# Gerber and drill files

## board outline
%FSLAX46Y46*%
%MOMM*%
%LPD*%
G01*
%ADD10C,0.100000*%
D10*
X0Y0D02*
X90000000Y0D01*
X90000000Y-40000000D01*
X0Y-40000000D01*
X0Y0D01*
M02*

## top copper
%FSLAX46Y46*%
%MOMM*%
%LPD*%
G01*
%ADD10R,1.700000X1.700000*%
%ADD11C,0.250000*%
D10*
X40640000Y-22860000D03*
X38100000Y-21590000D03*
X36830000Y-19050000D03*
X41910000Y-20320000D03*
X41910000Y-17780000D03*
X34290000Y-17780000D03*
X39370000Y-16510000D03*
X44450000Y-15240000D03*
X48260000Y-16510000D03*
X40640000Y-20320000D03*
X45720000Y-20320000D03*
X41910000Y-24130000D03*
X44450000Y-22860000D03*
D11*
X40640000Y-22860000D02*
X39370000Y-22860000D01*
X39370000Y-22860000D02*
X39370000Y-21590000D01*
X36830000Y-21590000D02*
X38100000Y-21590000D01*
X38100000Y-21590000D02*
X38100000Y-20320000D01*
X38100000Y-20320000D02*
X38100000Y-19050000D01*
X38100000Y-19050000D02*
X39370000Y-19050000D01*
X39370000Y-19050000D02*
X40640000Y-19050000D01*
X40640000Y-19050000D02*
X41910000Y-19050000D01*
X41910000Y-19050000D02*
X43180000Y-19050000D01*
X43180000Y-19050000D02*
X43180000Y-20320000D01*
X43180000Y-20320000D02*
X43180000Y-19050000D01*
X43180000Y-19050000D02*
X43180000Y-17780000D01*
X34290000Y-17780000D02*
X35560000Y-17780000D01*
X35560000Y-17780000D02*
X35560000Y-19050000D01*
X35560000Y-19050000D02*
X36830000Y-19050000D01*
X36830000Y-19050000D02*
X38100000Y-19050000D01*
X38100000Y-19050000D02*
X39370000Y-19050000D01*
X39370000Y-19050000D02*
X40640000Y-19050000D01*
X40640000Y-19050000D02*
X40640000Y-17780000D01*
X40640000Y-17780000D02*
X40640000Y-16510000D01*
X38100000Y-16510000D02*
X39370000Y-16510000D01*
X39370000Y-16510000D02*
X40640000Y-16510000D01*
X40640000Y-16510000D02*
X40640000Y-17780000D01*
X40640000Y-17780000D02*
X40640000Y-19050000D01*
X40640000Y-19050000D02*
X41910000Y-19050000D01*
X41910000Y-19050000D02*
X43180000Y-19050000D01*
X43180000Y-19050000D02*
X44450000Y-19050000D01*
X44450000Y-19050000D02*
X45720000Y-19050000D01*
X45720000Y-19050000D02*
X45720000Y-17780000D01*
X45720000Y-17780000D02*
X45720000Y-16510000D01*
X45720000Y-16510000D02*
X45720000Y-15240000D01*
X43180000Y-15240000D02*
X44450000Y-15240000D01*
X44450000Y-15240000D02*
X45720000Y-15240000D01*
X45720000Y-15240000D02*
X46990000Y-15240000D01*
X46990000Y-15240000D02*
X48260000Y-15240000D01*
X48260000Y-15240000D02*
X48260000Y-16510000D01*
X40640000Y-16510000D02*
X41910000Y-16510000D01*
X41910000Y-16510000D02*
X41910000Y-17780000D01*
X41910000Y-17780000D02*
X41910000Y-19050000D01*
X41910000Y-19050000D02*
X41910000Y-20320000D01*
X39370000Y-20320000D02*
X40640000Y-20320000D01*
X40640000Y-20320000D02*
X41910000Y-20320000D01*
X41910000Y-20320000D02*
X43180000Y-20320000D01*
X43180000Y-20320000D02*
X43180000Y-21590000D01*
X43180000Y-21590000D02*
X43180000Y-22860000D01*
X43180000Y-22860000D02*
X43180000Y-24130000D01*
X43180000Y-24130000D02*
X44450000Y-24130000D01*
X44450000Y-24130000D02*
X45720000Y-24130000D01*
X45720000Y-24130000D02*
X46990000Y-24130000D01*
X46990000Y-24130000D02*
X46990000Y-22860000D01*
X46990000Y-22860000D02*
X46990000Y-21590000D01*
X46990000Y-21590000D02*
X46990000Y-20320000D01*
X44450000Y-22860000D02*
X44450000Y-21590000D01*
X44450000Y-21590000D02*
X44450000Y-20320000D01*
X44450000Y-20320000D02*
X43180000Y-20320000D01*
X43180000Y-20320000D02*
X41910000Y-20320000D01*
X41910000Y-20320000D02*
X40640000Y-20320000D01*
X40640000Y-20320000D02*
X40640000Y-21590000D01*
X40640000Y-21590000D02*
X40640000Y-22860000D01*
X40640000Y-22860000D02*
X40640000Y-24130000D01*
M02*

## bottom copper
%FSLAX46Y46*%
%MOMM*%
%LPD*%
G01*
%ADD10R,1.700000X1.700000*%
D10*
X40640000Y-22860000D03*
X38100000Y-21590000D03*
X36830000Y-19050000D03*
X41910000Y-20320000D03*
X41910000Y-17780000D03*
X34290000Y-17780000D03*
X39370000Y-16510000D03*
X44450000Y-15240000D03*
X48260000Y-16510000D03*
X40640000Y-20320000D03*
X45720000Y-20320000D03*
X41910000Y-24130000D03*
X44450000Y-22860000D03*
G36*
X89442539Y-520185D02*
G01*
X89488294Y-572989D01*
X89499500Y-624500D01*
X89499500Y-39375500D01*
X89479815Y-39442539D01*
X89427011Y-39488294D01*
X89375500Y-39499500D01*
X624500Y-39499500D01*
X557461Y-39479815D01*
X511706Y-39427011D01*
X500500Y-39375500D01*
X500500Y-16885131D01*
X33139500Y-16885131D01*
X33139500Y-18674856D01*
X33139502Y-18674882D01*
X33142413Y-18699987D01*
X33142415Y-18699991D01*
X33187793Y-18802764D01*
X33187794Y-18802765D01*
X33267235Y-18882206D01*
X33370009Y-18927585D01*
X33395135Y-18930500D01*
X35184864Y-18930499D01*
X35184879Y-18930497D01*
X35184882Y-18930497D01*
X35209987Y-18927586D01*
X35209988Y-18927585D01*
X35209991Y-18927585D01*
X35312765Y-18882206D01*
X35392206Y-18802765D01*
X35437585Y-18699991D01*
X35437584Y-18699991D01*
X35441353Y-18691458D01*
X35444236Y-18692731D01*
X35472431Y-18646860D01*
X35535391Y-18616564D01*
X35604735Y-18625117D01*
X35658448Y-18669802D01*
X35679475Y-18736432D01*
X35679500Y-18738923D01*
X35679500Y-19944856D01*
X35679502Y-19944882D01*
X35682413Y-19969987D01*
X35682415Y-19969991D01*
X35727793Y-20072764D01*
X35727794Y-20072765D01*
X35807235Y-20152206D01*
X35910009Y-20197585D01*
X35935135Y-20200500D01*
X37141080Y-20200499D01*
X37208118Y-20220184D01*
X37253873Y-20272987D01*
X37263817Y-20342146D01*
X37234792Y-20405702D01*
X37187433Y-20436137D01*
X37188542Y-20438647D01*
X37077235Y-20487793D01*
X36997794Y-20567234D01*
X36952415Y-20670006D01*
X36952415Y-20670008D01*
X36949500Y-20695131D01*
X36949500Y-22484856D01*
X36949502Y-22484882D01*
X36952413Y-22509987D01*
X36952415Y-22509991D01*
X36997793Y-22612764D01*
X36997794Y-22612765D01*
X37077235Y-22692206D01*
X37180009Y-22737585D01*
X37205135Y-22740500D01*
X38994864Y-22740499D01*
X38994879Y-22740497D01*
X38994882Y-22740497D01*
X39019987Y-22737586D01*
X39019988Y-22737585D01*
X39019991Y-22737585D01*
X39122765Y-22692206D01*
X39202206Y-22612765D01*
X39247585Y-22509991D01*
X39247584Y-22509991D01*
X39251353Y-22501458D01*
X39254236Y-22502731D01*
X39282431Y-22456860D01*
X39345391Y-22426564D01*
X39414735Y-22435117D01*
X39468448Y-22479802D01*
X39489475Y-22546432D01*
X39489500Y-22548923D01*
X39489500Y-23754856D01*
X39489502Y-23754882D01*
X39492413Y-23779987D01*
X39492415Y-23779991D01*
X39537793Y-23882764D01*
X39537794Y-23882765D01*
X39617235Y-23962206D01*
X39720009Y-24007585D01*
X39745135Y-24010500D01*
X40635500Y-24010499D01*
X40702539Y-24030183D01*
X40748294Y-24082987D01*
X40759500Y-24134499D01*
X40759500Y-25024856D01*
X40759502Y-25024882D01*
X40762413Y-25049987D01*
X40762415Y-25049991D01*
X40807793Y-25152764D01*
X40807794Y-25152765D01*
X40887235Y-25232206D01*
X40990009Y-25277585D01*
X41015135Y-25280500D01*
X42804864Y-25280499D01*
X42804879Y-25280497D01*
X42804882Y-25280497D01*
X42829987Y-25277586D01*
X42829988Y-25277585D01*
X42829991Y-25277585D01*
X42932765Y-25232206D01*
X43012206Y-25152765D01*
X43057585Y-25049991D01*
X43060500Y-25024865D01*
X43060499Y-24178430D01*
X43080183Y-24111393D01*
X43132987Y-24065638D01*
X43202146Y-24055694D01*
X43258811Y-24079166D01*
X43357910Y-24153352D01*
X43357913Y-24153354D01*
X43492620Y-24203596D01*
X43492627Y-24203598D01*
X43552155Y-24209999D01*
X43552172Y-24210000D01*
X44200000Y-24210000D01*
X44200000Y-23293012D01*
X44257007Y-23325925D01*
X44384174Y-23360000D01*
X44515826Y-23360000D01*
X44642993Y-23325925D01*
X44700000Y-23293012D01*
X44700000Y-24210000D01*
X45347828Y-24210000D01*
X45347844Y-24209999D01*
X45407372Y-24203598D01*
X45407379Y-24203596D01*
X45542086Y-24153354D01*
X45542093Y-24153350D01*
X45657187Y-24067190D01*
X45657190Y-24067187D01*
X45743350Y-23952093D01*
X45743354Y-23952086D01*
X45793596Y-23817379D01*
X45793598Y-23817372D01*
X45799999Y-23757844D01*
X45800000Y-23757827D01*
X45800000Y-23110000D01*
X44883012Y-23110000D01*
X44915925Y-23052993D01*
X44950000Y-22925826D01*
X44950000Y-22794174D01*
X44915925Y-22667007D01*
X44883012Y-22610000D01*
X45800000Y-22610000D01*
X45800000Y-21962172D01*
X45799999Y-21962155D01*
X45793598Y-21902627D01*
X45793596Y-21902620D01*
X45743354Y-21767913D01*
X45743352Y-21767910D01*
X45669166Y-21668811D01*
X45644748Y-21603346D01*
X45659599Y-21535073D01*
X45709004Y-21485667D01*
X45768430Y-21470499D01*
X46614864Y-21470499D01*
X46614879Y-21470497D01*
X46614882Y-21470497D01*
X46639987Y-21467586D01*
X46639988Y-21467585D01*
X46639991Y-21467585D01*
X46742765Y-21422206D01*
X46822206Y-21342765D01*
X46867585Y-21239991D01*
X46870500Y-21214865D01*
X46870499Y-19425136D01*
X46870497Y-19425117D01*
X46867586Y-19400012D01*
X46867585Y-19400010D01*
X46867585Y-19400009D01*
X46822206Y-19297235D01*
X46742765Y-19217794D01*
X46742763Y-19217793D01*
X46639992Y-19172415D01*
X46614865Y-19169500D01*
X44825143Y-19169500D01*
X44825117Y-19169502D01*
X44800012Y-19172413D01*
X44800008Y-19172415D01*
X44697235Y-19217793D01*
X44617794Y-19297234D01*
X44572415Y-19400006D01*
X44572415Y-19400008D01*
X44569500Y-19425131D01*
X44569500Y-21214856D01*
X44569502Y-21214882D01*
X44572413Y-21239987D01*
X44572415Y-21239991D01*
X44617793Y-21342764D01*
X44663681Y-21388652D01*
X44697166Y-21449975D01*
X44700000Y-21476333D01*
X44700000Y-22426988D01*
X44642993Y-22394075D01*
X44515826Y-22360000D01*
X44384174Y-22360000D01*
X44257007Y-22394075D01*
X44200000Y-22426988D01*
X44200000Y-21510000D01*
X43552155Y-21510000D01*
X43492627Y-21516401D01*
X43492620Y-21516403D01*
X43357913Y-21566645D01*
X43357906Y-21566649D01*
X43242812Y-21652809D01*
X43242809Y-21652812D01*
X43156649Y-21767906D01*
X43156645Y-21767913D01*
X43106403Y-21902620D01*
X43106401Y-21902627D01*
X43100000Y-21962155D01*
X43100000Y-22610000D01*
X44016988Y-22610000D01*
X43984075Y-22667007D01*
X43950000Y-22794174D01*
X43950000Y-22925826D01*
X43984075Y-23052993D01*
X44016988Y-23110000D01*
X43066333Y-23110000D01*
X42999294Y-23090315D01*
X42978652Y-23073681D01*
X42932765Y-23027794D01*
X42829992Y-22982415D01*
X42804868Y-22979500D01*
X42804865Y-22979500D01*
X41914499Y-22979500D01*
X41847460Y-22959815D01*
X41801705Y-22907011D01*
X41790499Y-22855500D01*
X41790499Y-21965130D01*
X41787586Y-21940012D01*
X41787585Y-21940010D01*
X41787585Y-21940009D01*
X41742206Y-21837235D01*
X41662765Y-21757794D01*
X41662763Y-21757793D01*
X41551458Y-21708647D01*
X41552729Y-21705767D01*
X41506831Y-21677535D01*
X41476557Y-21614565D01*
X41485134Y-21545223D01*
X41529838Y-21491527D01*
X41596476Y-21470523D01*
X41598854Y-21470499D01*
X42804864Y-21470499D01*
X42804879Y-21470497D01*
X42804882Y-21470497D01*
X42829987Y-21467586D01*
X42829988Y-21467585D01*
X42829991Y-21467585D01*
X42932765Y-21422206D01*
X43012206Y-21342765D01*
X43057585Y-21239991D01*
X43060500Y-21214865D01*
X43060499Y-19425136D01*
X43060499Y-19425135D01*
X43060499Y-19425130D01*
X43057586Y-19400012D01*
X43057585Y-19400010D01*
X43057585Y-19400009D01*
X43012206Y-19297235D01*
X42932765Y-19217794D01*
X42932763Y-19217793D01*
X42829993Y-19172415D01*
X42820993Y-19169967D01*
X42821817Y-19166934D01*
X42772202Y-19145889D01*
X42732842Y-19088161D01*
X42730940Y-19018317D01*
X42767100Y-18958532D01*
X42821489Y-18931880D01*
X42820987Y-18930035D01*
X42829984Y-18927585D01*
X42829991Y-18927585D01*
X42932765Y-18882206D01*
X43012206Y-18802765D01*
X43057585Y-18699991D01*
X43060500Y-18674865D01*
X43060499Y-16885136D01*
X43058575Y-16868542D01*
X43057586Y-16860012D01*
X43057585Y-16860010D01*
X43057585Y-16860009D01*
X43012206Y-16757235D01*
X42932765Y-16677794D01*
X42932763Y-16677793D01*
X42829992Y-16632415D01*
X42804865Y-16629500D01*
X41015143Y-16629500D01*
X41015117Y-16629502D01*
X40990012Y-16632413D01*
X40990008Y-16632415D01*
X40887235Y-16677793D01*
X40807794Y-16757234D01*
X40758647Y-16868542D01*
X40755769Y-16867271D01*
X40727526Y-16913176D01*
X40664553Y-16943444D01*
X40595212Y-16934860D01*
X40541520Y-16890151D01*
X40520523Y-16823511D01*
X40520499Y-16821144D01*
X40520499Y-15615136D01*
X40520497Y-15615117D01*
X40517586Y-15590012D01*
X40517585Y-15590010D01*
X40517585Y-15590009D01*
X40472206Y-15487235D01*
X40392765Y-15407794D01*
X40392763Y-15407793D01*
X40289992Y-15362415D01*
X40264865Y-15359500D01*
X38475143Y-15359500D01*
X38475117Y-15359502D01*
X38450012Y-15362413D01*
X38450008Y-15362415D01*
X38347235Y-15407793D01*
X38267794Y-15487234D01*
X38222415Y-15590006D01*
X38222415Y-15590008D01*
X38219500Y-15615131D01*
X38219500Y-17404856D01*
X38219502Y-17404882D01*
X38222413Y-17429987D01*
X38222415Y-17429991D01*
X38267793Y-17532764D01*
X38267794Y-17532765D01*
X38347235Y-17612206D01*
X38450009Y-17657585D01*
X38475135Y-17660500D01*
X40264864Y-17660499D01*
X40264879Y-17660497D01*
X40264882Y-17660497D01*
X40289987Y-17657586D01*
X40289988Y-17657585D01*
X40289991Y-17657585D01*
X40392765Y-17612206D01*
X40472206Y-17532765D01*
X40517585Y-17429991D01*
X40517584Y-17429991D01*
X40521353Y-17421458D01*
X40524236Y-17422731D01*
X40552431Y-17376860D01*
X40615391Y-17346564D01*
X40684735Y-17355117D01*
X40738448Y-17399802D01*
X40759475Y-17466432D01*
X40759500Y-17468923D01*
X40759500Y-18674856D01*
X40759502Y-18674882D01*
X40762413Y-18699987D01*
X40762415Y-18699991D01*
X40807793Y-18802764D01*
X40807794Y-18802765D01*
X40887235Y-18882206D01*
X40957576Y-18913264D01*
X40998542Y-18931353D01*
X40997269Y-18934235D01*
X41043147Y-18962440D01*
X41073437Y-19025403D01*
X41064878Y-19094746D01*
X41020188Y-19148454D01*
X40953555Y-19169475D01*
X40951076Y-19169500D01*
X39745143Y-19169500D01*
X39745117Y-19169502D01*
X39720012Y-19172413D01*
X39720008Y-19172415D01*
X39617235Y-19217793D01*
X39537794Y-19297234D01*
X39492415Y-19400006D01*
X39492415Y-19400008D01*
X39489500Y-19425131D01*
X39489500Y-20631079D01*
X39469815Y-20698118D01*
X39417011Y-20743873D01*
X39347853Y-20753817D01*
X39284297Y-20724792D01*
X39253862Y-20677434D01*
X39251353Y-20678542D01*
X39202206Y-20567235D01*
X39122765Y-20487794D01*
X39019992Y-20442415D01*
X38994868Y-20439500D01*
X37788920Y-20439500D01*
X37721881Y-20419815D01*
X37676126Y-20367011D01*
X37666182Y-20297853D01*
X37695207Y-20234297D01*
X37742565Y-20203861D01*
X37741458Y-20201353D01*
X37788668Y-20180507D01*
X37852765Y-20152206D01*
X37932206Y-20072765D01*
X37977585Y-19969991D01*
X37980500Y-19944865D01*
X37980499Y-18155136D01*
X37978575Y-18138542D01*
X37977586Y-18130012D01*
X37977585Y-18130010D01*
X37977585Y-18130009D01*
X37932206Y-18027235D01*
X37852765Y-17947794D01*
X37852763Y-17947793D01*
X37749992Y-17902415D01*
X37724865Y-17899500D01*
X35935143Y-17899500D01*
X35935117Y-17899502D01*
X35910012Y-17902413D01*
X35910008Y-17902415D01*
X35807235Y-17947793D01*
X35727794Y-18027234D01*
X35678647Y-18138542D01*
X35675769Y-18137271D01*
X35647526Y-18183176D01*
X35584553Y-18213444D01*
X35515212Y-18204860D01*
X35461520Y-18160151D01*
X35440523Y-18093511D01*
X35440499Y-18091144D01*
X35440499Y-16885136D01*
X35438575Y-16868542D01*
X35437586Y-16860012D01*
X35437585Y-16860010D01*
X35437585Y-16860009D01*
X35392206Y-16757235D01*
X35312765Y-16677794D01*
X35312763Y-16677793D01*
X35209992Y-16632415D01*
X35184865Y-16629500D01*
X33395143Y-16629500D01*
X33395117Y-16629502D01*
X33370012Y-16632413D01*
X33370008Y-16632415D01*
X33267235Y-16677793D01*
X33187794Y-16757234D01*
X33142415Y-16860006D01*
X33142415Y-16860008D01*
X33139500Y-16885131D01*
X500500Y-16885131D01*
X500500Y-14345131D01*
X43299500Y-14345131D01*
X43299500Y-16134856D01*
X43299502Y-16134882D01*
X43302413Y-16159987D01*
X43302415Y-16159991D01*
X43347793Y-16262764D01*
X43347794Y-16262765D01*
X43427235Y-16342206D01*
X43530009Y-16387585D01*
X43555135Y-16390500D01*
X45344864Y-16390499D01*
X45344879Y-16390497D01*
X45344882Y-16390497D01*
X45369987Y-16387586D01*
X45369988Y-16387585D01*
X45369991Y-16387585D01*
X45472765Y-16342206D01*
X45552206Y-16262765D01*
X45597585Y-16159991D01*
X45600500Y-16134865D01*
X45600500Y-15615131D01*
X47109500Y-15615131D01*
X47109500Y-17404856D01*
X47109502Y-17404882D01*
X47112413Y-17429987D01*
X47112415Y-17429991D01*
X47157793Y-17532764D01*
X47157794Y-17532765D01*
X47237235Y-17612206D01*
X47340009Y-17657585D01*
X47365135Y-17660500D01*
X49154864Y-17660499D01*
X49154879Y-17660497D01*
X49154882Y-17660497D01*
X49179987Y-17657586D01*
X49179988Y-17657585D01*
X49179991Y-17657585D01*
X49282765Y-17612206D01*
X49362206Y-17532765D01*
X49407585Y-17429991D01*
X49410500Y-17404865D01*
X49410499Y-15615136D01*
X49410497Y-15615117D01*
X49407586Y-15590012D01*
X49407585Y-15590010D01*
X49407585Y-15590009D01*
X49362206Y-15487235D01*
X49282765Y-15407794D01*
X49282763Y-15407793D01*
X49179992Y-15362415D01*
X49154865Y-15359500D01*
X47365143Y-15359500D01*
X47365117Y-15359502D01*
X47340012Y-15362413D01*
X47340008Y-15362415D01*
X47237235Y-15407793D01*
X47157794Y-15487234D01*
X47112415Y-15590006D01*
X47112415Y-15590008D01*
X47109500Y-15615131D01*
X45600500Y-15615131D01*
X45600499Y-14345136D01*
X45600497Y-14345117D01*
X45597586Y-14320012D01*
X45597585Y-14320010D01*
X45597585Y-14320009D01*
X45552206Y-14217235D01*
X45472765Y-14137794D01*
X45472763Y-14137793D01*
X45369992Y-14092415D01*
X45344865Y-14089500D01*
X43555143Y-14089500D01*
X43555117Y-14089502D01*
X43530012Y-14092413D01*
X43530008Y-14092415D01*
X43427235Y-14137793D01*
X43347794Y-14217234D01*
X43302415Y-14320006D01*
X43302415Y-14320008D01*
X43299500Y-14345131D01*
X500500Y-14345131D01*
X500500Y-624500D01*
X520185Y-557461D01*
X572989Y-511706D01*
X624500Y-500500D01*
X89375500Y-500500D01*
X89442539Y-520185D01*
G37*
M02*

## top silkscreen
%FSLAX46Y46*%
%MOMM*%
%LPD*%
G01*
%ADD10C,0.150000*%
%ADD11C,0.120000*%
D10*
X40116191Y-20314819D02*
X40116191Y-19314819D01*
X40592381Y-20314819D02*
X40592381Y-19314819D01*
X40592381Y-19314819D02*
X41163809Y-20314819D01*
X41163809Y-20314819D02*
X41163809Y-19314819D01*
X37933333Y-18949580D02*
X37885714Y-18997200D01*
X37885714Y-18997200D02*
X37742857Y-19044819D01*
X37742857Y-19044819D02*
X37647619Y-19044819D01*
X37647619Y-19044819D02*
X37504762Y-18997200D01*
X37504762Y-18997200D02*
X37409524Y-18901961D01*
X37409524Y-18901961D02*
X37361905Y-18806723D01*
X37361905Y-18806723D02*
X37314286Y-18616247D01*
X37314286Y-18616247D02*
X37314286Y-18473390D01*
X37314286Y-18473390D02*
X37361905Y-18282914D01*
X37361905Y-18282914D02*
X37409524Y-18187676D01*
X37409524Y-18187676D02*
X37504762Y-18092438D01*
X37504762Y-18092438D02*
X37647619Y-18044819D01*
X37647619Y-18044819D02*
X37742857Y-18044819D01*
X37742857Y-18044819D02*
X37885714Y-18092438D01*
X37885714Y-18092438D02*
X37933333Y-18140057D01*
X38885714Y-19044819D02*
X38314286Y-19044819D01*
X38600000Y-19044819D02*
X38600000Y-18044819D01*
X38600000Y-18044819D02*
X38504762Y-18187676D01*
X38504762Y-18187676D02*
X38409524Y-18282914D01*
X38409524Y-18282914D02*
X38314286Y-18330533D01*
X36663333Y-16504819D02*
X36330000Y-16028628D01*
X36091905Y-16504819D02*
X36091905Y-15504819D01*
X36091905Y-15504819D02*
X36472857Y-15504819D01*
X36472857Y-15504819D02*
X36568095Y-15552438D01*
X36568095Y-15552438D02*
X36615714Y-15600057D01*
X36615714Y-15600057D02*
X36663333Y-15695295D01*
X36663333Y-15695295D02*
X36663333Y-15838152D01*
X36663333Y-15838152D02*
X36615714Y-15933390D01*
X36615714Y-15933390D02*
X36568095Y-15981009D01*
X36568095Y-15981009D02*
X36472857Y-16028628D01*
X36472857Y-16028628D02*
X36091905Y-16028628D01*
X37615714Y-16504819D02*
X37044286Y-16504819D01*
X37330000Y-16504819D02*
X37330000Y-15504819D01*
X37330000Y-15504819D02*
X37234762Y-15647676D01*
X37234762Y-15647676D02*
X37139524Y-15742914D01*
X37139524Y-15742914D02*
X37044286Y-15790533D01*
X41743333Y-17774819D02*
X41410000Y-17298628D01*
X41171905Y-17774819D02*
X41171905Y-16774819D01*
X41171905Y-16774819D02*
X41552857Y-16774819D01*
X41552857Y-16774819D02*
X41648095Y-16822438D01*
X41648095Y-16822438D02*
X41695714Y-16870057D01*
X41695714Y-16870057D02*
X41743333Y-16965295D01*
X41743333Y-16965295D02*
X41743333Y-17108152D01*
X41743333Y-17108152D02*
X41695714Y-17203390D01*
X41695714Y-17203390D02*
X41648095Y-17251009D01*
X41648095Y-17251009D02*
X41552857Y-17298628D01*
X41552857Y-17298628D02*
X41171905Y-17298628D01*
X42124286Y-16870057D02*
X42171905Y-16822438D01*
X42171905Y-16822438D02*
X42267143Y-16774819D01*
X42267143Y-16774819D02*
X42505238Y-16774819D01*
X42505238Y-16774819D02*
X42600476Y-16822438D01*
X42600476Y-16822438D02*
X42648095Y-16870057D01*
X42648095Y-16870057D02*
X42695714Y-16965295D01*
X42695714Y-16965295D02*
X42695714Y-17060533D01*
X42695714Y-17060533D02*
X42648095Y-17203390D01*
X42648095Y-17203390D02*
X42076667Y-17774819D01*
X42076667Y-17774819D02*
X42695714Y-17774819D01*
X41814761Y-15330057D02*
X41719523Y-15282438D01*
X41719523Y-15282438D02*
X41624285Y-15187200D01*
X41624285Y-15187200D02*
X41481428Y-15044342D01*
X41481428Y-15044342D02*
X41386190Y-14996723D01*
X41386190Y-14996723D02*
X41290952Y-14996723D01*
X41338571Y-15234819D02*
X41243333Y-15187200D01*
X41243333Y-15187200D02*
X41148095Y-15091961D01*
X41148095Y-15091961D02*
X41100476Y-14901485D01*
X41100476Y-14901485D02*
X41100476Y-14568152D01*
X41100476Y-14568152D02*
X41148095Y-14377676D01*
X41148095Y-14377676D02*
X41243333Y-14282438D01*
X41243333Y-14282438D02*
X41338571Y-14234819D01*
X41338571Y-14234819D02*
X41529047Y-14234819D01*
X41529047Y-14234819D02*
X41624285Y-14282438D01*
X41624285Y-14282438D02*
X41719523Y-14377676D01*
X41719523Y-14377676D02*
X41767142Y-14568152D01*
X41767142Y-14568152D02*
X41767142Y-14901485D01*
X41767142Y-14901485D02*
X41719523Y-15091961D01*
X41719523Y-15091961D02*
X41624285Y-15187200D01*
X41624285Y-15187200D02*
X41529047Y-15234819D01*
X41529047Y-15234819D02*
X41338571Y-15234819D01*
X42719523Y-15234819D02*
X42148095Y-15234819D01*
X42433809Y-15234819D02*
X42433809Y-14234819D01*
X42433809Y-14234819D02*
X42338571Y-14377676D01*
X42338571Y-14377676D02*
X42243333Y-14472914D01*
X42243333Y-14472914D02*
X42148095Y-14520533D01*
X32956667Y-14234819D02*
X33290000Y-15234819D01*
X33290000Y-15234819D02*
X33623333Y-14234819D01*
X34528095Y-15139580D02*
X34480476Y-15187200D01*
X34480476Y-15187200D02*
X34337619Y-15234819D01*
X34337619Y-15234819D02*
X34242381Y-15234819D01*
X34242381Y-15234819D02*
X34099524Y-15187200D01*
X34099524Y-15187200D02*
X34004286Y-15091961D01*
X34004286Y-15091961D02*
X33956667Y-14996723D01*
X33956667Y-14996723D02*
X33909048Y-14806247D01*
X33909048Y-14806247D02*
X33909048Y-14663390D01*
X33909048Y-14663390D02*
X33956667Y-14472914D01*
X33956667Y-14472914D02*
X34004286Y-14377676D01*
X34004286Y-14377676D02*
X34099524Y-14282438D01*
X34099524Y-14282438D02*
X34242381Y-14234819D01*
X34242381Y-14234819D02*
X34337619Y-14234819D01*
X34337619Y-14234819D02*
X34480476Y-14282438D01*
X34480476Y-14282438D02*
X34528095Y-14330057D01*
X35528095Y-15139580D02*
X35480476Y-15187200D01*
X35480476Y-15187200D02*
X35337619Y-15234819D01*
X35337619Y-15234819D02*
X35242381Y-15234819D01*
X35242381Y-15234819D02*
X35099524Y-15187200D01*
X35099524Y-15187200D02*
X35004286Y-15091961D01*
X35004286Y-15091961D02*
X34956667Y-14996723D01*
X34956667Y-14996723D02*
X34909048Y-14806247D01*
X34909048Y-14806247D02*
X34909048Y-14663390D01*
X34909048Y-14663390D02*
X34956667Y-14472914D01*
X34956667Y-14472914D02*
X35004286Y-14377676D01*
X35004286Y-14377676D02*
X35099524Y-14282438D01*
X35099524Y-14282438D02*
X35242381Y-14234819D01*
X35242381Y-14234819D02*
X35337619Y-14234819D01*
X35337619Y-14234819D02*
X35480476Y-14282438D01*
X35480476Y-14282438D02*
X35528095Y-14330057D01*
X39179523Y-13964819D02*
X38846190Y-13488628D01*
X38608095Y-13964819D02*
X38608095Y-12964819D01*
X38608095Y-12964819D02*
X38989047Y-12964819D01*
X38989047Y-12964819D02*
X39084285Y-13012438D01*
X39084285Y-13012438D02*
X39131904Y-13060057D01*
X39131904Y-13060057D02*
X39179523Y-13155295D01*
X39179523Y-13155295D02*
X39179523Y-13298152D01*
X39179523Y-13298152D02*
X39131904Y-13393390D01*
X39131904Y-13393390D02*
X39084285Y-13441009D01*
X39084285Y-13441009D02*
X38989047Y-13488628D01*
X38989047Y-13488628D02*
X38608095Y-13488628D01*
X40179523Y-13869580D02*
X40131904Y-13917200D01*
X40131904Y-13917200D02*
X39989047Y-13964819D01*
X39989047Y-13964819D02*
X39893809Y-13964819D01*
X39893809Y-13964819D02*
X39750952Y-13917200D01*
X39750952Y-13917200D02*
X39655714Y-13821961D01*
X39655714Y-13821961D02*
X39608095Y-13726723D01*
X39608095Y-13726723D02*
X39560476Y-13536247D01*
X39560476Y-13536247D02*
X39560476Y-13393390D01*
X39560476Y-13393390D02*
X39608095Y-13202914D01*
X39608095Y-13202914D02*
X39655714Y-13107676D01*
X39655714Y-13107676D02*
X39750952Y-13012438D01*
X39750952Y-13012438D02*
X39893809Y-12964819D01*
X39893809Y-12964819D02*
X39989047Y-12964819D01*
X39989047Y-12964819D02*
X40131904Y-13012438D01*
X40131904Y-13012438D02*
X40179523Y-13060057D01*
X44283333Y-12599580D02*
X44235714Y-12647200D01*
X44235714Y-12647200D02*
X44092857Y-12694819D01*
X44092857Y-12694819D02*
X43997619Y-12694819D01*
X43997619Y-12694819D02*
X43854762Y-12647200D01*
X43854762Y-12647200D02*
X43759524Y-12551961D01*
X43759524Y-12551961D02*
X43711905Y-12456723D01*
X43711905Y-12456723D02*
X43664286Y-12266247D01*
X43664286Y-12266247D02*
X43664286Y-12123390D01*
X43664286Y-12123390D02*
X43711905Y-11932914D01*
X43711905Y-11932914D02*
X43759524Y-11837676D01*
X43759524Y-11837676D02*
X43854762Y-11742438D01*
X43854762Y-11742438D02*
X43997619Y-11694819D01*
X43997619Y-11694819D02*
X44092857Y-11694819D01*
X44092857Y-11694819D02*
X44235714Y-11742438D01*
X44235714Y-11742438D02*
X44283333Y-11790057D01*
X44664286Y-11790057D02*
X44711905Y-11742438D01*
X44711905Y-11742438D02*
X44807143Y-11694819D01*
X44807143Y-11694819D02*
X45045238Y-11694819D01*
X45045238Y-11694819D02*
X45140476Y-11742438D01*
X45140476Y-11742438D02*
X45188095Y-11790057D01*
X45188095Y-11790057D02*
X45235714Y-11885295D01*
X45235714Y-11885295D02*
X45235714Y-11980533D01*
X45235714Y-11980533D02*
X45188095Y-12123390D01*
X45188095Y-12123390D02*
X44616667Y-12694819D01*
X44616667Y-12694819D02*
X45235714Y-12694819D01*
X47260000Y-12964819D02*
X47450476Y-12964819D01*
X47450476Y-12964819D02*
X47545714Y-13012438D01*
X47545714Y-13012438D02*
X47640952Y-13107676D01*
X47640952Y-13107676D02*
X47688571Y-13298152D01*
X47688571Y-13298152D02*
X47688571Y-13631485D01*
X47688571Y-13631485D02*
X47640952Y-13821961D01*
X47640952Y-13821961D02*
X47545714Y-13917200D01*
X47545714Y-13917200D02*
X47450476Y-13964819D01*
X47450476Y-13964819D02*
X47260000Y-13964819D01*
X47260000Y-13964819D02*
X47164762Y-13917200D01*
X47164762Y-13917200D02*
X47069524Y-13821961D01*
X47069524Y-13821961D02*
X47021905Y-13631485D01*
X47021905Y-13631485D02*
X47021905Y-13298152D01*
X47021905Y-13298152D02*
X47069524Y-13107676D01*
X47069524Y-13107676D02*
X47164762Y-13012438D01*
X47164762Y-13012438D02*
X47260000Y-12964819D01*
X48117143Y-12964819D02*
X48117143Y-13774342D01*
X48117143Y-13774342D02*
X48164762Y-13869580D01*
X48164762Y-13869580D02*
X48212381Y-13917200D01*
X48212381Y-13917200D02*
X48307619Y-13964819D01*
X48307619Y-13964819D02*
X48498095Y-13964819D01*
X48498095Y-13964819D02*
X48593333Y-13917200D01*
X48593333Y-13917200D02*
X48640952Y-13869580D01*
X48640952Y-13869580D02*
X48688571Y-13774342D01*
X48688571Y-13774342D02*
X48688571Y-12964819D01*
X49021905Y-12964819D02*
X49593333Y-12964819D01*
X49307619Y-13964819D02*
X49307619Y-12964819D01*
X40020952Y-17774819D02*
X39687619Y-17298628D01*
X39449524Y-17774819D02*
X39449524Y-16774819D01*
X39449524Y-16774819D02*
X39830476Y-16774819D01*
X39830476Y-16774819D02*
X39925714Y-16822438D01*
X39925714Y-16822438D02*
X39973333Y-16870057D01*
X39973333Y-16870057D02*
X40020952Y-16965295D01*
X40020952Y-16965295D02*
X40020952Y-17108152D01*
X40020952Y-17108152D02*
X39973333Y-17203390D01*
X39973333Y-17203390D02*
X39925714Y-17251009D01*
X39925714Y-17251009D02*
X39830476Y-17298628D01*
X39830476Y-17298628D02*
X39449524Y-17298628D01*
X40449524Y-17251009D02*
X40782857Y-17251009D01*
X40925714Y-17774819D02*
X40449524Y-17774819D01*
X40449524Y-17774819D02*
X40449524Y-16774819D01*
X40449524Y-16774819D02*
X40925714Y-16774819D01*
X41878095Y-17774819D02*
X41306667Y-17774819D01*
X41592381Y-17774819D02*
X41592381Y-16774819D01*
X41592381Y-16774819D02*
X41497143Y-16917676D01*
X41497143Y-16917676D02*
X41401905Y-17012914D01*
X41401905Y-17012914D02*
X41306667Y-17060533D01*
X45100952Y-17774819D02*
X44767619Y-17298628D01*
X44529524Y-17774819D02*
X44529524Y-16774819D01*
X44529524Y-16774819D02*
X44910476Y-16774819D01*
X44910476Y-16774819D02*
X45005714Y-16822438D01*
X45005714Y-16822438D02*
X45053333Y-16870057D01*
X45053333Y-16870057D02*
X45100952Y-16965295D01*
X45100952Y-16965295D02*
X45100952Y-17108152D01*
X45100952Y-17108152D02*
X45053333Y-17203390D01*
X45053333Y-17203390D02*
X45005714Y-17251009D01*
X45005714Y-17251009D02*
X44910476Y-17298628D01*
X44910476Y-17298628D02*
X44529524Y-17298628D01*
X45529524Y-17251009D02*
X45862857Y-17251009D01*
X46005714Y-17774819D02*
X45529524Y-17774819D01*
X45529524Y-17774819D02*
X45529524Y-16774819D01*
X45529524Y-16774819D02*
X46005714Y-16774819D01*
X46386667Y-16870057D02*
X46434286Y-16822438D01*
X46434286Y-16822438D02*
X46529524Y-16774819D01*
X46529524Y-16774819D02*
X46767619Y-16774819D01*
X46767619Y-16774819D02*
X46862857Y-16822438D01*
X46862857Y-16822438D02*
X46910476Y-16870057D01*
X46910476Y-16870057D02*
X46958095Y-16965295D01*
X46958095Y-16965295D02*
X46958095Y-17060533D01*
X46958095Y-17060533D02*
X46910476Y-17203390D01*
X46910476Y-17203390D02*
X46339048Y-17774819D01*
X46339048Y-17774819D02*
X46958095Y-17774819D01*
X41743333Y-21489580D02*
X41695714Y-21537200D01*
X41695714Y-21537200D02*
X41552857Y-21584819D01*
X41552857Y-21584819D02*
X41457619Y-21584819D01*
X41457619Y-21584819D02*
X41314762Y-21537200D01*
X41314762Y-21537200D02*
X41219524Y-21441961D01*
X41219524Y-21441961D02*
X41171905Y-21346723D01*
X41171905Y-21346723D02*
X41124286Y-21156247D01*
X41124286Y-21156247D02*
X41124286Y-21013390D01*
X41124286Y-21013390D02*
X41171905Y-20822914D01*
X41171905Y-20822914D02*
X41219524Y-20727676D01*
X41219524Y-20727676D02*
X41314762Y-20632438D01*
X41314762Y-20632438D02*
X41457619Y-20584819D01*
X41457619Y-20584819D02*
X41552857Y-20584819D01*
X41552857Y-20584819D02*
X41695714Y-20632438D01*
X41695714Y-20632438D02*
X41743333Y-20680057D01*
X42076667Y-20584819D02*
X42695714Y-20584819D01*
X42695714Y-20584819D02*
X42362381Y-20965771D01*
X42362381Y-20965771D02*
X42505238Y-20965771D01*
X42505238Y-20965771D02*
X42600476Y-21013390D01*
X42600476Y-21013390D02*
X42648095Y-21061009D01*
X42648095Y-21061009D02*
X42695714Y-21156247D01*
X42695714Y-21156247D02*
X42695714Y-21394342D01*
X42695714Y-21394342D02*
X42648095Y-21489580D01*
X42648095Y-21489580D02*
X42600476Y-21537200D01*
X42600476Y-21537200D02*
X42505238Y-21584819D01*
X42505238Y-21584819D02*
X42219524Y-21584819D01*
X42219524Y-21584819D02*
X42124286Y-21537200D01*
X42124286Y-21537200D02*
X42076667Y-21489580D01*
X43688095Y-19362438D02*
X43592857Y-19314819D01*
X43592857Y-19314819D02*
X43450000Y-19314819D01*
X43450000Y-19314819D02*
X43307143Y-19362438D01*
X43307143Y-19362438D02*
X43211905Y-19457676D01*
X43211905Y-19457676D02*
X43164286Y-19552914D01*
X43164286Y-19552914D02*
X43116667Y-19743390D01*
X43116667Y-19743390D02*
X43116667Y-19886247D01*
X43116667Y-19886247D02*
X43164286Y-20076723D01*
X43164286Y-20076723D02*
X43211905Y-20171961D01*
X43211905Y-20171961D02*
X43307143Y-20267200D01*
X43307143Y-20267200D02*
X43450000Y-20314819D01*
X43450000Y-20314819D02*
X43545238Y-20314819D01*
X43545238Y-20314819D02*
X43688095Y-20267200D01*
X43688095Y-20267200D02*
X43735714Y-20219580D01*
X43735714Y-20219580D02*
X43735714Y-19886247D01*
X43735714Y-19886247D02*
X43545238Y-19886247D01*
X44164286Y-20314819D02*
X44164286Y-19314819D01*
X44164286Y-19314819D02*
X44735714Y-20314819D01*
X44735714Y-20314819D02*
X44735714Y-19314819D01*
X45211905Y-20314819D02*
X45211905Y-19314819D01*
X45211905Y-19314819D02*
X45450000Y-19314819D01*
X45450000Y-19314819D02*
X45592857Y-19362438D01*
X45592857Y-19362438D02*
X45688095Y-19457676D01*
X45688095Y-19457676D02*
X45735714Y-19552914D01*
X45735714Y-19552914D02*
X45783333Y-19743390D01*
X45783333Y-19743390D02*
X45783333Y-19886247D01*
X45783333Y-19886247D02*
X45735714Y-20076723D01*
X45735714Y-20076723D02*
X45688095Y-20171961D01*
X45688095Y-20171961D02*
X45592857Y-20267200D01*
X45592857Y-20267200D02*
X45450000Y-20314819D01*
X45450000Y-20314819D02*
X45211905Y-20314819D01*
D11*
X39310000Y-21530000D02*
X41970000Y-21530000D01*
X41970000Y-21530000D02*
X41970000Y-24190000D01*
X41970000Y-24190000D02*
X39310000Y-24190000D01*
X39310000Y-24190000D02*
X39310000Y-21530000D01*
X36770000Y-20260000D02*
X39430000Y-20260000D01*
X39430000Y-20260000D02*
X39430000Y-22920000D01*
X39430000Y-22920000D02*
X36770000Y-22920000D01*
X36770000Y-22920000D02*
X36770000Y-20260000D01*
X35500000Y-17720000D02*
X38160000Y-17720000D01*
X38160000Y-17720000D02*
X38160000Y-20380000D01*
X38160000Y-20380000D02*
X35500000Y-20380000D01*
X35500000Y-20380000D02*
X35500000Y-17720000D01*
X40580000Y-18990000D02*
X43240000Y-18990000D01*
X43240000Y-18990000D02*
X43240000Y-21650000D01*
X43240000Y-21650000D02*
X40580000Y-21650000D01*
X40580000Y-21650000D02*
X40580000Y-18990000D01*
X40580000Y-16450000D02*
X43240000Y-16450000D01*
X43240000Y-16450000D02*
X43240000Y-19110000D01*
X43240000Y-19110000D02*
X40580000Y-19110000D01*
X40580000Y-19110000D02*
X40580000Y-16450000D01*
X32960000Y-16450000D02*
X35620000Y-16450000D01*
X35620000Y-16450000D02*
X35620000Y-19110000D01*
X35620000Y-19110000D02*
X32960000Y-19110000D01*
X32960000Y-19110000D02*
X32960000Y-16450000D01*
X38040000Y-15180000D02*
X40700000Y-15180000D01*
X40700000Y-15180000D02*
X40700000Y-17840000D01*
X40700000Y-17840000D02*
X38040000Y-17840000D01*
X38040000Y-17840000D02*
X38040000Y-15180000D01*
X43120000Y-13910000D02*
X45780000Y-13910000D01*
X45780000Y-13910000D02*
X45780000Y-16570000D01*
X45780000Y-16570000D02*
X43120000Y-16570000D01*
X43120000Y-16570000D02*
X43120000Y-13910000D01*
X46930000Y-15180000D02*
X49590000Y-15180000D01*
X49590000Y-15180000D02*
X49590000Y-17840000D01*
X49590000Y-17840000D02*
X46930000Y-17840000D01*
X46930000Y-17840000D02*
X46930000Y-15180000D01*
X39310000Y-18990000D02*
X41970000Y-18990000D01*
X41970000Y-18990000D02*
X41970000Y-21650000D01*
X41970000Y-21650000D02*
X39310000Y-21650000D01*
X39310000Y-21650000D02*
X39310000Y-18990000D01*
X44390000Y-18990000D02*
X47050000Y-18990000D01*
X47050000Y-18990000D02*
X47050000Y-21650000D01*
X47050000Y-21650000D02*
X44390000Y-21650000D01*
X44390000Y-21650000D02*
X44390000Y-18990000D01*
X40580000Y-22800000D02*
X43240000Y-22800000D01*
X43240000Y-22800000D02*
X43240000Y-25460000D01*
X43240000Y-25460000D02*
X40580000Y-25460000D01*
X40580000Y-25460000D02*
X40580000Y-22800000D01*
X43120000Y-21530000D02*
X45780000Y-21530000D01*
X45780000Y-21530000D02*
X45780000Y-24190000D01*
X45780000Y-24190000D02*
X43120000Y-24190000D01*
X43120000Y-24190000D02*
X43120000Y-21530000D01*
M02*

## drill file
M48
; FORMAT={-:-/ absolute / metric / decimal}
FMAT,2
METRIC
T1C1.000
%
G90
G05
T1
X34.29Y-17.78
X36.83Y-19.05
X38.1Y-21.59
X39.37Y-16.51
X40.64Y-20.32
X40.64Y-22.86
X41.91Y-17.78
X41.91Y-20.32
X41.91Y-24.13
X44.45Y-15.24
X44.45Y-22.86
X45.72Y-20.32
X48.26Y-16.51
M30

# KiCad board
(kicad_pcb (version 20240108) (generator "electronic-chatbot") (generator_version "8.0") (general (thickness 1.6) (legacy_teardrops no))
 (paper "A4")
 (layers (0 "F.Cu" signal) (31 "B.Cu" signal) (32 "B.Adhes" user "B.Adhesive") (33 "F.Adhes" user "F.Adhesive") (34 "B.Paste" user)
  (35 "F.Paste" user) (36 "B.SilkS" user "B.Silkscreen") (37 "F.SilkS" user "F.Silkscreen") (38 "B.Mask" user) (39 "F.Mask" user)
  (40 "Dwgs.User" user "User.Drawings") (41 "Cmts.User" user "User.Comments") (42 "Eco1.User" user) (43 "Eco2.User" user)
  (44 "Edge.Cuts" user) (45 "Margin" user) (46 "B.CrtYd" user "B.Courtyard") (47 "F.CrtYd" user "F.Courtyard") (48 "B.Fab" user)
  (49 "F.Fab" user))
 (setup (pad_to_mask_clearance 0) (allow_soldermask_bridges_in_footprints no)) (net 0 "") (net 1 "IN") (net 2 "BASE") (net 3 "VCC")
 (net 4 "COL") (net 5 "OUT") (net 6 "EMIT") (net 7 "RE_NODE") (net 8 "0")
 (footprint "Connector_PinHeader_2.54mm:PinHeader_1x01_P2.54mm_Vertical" (layer "F.Cu") (at 40.64 22.86)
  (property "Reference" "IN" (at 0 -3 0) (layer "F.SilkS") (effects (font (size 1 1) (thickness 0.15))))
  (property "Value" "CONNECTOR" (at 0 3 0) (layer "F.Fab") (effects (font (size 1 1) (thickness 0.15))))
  (fp_line (start -1.33 -1.33) (end 1.33 -1.33) (stroke (width 0.12) (type solid)) (layer "F.SilkS"))
  (fp_line (start 1.33 -1.33) (end 1.33 1.33) (stroke (width 0.12) (type solid)) (layer "F.SilkS"))
  (fp_line (start 1.33 1.33) (end -1.33 1.33) (stroke (width 0.12) (type solid)) (layer "F.SilkS"))
  (fp_line (start -1.33 1.33) (end -1.33 -1.33) (stroke (width 0.12) (type solid)) (layer "F.SilkS"))
  (pad "1" thru_hole rect (at 0 0) (size 1.7 1.7) (drill 1.0) (layers "*.Cu" "*.Mask") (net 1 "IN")))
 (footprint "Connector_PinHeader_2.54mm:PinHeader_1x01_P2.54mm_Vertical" (layer "F.Cu") (at 38.1 21.59)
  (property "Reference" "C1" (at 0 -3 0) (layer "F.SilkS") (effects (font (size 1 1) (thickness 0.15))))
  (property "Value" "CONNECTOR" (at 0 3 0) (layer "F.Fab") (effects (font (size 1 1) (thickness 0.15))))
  (fp_line (start -1.33 -1.33) (end 1.33 -1.33) (stroke (width 0.12) (type solid)) (layer "F.SilkS"))
  (fp_line (start 1.33 -1.33) (end 1.33 1.33) (stroke (width 0.12) (type solid)) (layer "F.SilkS"))
  (fp_line (start 1.33 1.33) (end -1.33 1.33) (stroke (width 0.12) (type solid)) (layer "F.SilkS"))
  (fp_line (start -1.33 1.33) (end -1.33 -1.33) (stroke (width 0.12) (type solid)) (layer "F.SilkS"))
  (pad "1" thru_hole rect (at 0 0) (size 1.7 1.7) (drill 1.0) (layers "*.Cu" "*.Mask") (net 1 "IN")))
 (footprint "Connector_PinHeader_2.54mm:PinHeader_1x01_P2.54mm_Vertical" (layer "F.Cu") (at 36.83 19.05)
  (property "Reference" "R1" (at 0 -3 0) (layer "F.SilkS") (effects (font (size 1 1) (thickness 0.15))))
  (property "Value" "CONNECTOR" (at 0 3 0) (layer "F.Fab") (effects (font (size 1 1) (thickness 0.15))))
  (fp_line (start -1.33 -1.33) (end 1.33 -1.33) (stroke (width 0.12) (type solid)) (layer "F.SilkS"))
  (fp_line (start 1.33 -1.33) (end 1.33 1.33) (stroke (width 0.12) (type solid)) (layer "F.SilkS"))
  (fp_line (start 1.33 1.33) (end -1.33 1.33) (stroke (width 0.12) (type solid)) (layer "F.SilkS"))
  (fp_line (start -1.33 1.33) (end -1.33 -1.33) (stroke (width 0.12) (type solid)) (layer "F.SilkS"))
  (pad "1" thru_hole rect (at 0 0) (size 1.7 1.7) (drill 1.0) (layers "*.Cu" "*.Mask") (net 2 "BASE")))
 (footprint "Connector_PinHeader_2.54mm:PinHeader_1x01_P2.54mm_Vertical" (layer "F.Cu") (at 41.910000000000004 20.32)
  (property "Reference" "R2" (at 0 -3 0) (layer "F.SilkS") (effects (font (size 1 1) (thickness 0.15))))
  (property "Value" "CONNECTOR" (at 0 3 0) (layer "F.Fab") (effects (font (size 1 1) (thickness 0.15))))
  (fp_line (start -1.33 -1.33) (end 1.33 -1.33) (stroke (width 0.12) (type solid)) (layer "F.SilkS"))
  (fp_line (start 1.33 -1.33) (end 1.33 1.33) (stroke (width 0.12) (type solid)) (layer "F.SilkS"))
  (fp_line (start 1.33 1.33) (end -1.33 1.33) (stroke (width 0.12) (type solid)) (layer "F.SilkS"))
  (fp_line (start -1.33 1.33) (end -1.33 -1.33) (stroke (width 0.12) (type solid)) (layer "F.SilkS"))
  (pad "1" thru_hole rect (at 0 0) (size 1.7 1.7) (drill 1.0) (layers "*.Cu" "*.Mask") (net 2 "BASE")))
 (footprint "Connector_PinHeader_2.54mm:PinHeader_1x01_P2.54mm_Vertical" (layer "F.Cu") (at 41.910000000000004 17.78)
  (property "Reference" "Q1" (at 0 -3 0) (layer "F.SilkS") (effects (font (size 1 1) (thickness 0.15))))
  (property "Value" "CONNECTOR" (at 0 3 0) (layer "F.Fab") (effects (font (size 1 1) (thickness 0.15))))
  (fp_line (start -1.33 -1.33) (end 1.33 -1.33) (stroke (width 0.12) (type solid)) (layer "F.SilkS"))
  (fp_line (start 1.33 -1.33) (end 1.33 1.33) (stroke (width 0.12) (type solid)) (layer "F.SilkS"))
  (fp_line (start 1.33 1.33) (end -1.33 1.33) (stroke (width 0.12) (type solid)) (layer "F.SilkS"))
  (fp_line (start -1.33 1.33) (end -1.33 -1.33) (stroke (width 0.12) (type solid)) (layer "F.SilkS"))
  (pad "1" thru_hole rect (at 0 0) (size 1.7 1.7) (drill 1.0) (layers "*.Cu" "*.Mask") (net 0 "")))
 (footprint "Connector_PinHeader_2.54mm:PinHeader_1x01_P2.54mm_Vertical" (layer "F.Cu") (at 34.29 17.78)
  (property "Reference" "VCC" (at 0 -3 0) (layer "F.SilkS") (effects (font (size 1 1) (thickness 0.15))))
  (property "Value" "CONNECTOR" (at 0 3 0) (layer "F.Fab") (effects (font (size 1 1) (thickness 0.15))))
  (fp_line (start -1.33 -1.33) (end 1.33 -1.33) (stroke (width 0.12) (type solid)) (layer "F.SilkS"))
  (fp_line (start 1.33 -1.33) (end 1.33 1.33) (stroke (width 0.12) (type solid)) (layer "F.SilkS"))
  (fp_line (start 1.33 1.33) (end -1.33 1.33) (stroke (width 0.12) (type solid)) (layer "F.SilkS"))
  (fp_line (start -1.33 1.33) (end -1.33 -1.33) (stroke (width 0.12) (type solid)) (layer "F.SilkS"))
  (pad "1" thru_hole rect (at 0 0) (size 1.7 1.7) (drill 1.0) (layers "*.Cu" "*.Mask") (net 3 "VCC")))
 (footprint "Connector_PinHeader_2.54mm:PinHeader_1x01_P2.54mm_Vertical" (layer "F.Cu") (at 39.37 16.51)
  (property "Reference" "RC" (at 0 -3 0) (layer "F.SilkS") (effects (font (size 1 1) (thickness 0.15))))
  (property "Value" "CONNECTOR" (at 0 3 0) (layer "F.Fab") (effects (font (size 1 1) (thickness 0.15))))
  (fp_line (start -1.33 -1.33) (end 1.33 -1.33) (stroke (width 0.12) (type solid)) (layer "F.SilkS"))
  (fp_line (start 1.33 -1.33) (end 1.33 1.33) (stroke (width 0.12) (type solid)) (layer "F.SilkS"))
  (fp_line (start 1.33 1.33) (end -1.33 1.33) (stroke (width 0.12) (type solid)) (layer "F.SilkS"))
  (fp_line (start -1.33 1.33) (end -1.33 -1.33) (stroke (width 0.12) (type solid)) (layer "F.SilkS"))
  (pad "1" thru_hole rect (at 0 0) (size 1.7 1.7) (drill 1.0) (layers "*.Cu" "*.Mask") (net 3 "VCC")))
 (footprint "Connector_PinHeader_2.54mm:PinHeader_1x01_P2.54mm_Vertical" (layer "F.Cu") (at 44.45 15.24)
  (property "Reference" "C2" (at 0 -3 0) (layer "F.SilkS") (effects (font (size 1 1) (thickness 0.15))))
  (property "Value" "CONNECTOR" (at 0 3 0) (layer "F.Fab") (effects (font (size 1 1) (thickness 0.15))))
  (fp_line (start -1.33 -1.33) (end 1.33 -1.33) (stroke (width 0.12) (type solid)) (layer "F.SilkS"))
  (fp_line (start 1.33 -1.33) (end 1.33 1.33) (stroke (width 0.12) (type solid)) (layer "F.SilkS"))
  (fp_line (start 1.33 1.33) (end -1.33 1.33) (stroke (width 0.12) (type solid)) (layer "F.SilkS"))
  (fp_line (start -1.33 1.33) (end -1.33 -1.33) (stroke (width 0.12) (type solid)) (layer "F.SilkS"))
  (pad "1" thru_hole rect (at 0 0) (size 1.7 1.7) (drill 1.0) (layers "*.Cu" "*.Mask") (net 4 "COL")))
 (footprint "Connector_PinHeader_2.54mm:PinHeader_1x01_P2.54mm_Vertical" (layer "F.Cu") (at 48.26 16.51)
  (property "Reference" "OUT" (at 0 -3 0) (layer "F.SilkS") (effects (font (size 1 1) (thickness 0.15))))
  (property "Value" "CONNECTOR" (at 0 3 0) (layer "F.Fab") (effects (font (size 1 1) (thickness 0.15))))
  (fp_line (start -1.33 -1.33) (end 1.33 -1.33) (stroke (width 0.12) (type solid)) (layer "F.SilkS"))
  (fp_line (start 1.33 -1.33) (end 1.33 1.33) (stroke (width 0.12) (type solid)) (layer "F.SilkS"))
  (fp_line (start 1.33 1.33) (end -1.33 1.33) (stroke (width 0.12) (type solid)) (layer "F.SilkS"))
  (fp_line (start -1.33 1.33) (end -1.33 -1.33) (stroke (width 0.12) (type solid)) (layer "F.SilkS"))
  (pad "1" thru_hole rect (at 0 0) (size 1.7 1.7) (drill 1.0) (layers "*.Cu" "*.Mask") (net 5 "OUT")))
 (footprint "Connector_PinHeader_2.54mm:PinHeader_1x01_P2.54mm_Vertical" (layer "F.Cu") (at 40.64 20.32)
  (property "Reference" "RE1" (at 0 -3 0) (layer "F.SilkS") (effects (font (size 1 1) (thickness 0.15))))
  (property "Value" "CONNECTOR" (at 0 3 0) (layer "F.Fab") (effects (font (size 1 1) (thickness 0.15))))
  (fp_line (start -1.33 -1.33) (end 1.33 -1.33) (stroke (width 0.12) (type solid)) (layer "F.SilkS"))
  (fp_line (start 1.33 -1.33) (end 1.33 1.33) (stroke (width 0.12) (type solid)) (layer "F.SilkS"))
  (fp_line (start 1.33 1.33) (end -1.33 1.33) (stroke (width 0.12) (type solid)) (layer "F.SilkS"))
  (fp_line (start -1.33 1.33) (end -1.33 -1.33) (stroke (width 0.12) (type solid)) (layer "F.SilkS"))
  (pad "1" thru_hole rect (at 0 0) (size 1.7 1.7) (drill 1.0) (layers "*.Cu" "*.Mask") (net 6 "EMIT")))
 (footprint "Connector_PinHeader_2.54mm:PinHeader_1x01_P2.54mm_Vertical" (layer "F.Cu") (at 45.72 20.32)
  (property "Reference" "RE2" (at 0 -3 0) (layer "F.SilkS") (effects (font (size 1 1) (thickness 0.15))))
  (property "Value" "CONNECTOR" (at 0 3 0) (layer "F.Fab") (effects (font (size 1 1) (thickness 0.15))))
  (fp_line (start -1.33 -1.33) (end 1.33 -1.33) (stroke (width 0.12) (type solid)) (layer "F.SilkS"))
  (fp_line (start 1.33 -1.33) (end 1.33 1.33) (stroke (width 0.12) (type solid)) (layer "F.SilkS"))
  (fp_line (start 1.33 1.33) (end -1.33 1.33) (stroke (width 0.12) (type solid)) (layer "F.SilkS"))
  (fp_line (start -1.33 1.33) (end -1.33 -1.33) (stroke (width 0.12) (type solid)) (layer "F.SilkS"))
  (pad "1" thru_hole rect (at 0 0) (size 1.7 1.7) (drill 1.0) (layers "*.Cu" "*.Mask") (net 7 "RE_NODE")))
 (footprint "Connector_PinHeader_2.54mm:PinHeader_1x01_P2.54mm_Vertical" (layer "F.Cu") (at 41.910000000000004 24.13)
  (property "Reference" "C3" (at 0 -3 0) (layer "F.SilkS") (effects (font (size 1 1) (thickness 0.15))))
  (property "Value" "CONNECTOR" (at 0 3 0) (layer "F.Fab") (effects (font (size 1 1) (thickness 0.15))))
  (fp_line (start -1.33 -1.33) (end 1.33 -1.33) (stroke (width 0.12) (type solid)) (layer "F.SilkS"))
  (fp_line (start 1.33 -1.33) (end 1.33 1.33) (stroke (width 0.12) (type solid)) (layer "F.SilkS"))
  (fp_line (start 1.33 1.33) (end -1.33 1.33) (stroke (width 0.12) (type solid)) (layer "F.SilkS"))
  (fp_line (start -1.33 1.33) (end -1.33 -1.33) (stroke (width 0.12) (type solid)) (layer "F.SilkS"))
  (pad "1" thru_hole rect (at 0 0) (size 1.7 1.7) (drill 1.0) (layers "*.Cu" "*.Mask") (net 7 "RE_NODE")))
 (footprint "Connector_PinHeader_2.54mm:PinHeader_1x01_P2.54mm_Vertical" (layer "F.Cu") (at 44.45 22.86)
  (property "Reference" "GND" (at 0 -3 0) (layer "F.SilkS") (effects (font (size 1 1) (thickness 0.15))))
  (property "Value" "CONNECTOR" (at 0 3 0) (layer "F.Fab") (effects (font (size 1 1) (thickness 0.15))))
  (fp_line (start -1.33 -1.33) (end 1.33 -1.33) (stroke (width 0.12) (type solid)) (layer "F.SilkS"))
  (fp_line (start 1.33 -1.33) (end 1.33 1.33) (stroke (width 0.12) (type solid)) (layer "F.SilkS"))
  (fp_line (start 1.33 1.33) (end -1.33 1.33) (stroke (width 0.12) (type solid)) (layer "F.SilkS"))
  (fp_line (start -1.33 1.33) (end -1.33 -1.33) (stroke (width 0.12) (type solid)) (layer "F.SilkS"))
  (pad "1" thru_hole rect (at 0 0) (size 1.7 1.7) (drill 1.0) (layers "*.Cu" "*.Mask") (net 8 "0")))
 (gr_rect (start 0 0) (end 90.0 40.0) (layer "Edge.Cuts") (stroke (width 0.1) (type solid)) (fill none))
 (segment (start 40.64 22.86) (end 39.37 22.86) (width 0.25) (layer "F.Cu") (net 1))
 (segment (start 39.37 22.86) (end 39.37 21.59) (width 0.25) (layer "F.Cu") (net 1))
 (segment (start 36.83 21.59) (end 38.1 21.59) (width 0.25) (layer "F.Cu") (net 2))
 (segment (start 38.1 21.59) (end 38.1 20.32) (width 0.25) (layer "F.Cu") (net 2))
 (segment (start 38.1 20.32) (end 38.1 19.05) (width 0.25) (layer "F.Cu") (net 2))
 (segment (start 38.1 19.05) (end 39.37 19.05) (width 0.25) (layer "F.Cu") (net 2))
 (segment (start 39.37 19.05) (end 40.64 19.05) (width 0.25) (layer "F.Cu") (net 2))
 (segment (start 40.64 19.05) (end 41.91 19.05) (width 0.25) (layer "F.Cu") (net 2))
 (segment (start 41.91 19.05) (end 43.18 19.05) (width 0.25) (layer "F.Cu") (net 2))
 (segment (start 43.18 19.05) (end 43.18 20.32) (width 0.25) (layer "F.Cu") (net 2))
 (segment (start 43.18 20.32) (end 43.18 19.05) (width 0.25) (layer "F.Cu") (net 2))
 (segment (start 43.18 19.05) (end 43.18 17.78) (width 0.25) (layer "F.Cu") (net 2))
 (segment (start 34.29 17.78) (end 35.56 17.78) (width 0.25) (layer "F.Cu") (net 3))
 (segment (start 35.56 17.78) (end 35.56 19.05) (width 0.25) (layer "F.Cu") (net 3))
 (segment (start 35.56 19.05) (end 36.83 19.05) (width 0.25) (layer "F.Cu") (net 3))
 (segment (start 36.83 19.05) (end 38.1 19.05) (width 0.25) (layer "F.Cu") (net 3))
 (segment (start 38.1 19.05) (end 39.37 19.05) (width 0.25) (layer "F.Cu") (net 3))
 (segment (start 39.37 19.05) (end 40.64 19.05) (width 0.25) (layer "F.Cu") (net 3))
 (segment (start 40.64 19.05) (end 40.64 17.78) (width 0.25) (layer "F.Cu") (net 3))
 (segment (start 40.64 17.78) (end 40.64 16.51) (width 0.25) (layer "F.Cu") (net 3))
 (segment (start 38.1 16.51) (end 39.37 16.51) (width 0.25) (layer "F.Cu") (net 4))
 (segment (start 39.37 16.51) (end 40.64 16.51) (width 0.25) (layer "F.Cu") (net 4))
 (segment (start 40.64 16.51) (end 40.64 17.78) (width 0.25) (layer "F.Cu") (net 4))
 (segment (start 40.64 17.78) (end 40.64 19.05) (width 0.25) (layer "F.Cu") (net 4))
 (segment (start 40.64 19.05) (end 41.91 19.05) (width 0.25) (layer "F.Cu") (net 4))
 (segment (start 41.91 19.05) (end 43.18 19.05) (width 0.25) (layer "F.Cu") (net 4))
 (segment (start 43.18 19.05) (end 44.45 19.05) (width 0.25) (layer "F.Cu") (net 4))
 (segment (start 44.45 19.05) (end 45.72 19.05) (width 0.25) (layer "F.Cu") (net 4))
 (segment (start 45.72 19.05) (end 45.72 17.78) (width 0.25) (layer "F.Cu") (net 4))
 (segment (start 45.72 17.78) (end 45.72 16.51) (width 0.25) (layer "F.Cu") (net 4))
 (segment (start 45.72 16.51) (end 45.72 15.24) (width 0.25) (layer "F.Cu") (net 4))
 (segment (start 43.18 15.24) (end 44.45 15.24) (width 0.25) (layer "F.Cu") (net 5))
 (segment (start 44.45 15.24) (end 45.72 15.24) (width 0.25) (layer "F.Cu") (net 5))
 (segment (start 45.72 15.24) (end 46.99 15.24) (width 0.25) (layer "F.Cu") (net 5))
 (segment (start 46.99 15.24) (end 48.26 15.24) (width 0.25) (layer "F.Cu") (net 5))
 (segment (start 48.26 15.24) (end 48.26 16.51) (width 0.25) (layer "F.Cu") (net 5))
 (segment (start 40.64 16.51) (end 41.91 16.51) (width 0.25) (layer "F.Cu") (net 6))
 (segment (start 41.91 16.51) (end 41.91 17.78) (width 0.25) (layer "F.Cu") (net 6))
 (segment (start 41.91 17.78) (end 41.91 19.05) (width 0.25) (layer "F.Cu") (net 6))
 (segment (start 41.91 19.05) (end 41.91 20.32) (width 0.25) (layer "F.Cu") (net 6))
 (segment (start 39.37 20.32) (end 40.64 20.32) (width 0.25) (layer "F.Cu") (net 7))
 (segment (start 40.64 20.32) (end 41.91 20.32) (width 0.25) (layer "F.Cu") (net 7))
 (segment (start 41.91 20.32) (end 43.18 20.32) (width 0.25) (layer "F.Cu") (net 7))
 (segment (start 43.18 20.32) (end 43.18 21.59) (width 0.25) (layer "F.Cu") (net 7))
 (segment (start 43.18 21.59) (end 43.18 22.86) (width 0.25) (layer "F.Cu") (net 7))
 (segment (start 43.18 22.86) (end 43.18 24.13) (width 0.25) (layer "F.Cu") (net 7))
 (segment (start 43.18 24.13) (end 44.45 24.13) (width 0.25) (layer "F.Cu") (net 7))
 (segment (start 44.45 24.13) (end 45.72 24.13) (width 0.25) (layer "F.Cu") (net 7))
 (segment (start 45.72 24.13) (end 46.99 24.13) (width 0.25) (layer "F.Cu") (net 7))
 (segment (start 46.99 24.13) (end 46.99 22.86) (width 0.25) (layer "F.Cu") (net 7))
 (segment (start 46.99 22.86) (end 46.99 21.59) (width 0.25) (layer "F.Cu") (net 7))
 (segment (start 46.99 21.59) (end 46.99 20.32) (width 0.25) (layer "F.Cu") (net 7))
 (segment (start 44.45 22.86) (end 44.45 21.59) (width 0.25) (layer "F.Cu") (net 8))
 (segment (start 44.45 21.59) (end 44.45 20.32) (width 0.25) (layer "F.Cu") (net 8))
 (segment (start 44.45 20.32) (end 43.18 20.32) (width 0.25) (layer "F.Cu") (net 8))
 (segment (start 43.18 20.32) (end 41.91 20.32) (width 0.25) (layer "F.Cu") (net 8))
 (segment (start 41.91 20.32) (end 40.64 20.32) (width 0.25) (layer "F.Cu") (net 8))
 (segment (start 40.64 20.32) (end 40.64 21.59) (width 0.25) (layer "F.Cu") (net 8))
 (segment (start 40.64 21.59) (end 40.64 22.86) (width 0.25) (layer "F.Cu") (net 8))
 (segment (start 40.64 22.86) (end 40.64 24.13) (width 0.25) (layer "F.Cu") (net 8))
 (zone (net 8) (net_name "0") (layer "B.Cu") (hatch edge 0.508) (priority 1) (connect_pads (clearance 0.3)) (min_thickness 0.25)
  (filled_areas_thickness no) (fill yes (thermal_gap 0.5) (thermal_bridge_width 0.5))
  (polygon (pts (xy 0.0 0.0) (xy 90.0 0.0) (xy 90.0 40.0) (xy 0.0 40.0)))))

